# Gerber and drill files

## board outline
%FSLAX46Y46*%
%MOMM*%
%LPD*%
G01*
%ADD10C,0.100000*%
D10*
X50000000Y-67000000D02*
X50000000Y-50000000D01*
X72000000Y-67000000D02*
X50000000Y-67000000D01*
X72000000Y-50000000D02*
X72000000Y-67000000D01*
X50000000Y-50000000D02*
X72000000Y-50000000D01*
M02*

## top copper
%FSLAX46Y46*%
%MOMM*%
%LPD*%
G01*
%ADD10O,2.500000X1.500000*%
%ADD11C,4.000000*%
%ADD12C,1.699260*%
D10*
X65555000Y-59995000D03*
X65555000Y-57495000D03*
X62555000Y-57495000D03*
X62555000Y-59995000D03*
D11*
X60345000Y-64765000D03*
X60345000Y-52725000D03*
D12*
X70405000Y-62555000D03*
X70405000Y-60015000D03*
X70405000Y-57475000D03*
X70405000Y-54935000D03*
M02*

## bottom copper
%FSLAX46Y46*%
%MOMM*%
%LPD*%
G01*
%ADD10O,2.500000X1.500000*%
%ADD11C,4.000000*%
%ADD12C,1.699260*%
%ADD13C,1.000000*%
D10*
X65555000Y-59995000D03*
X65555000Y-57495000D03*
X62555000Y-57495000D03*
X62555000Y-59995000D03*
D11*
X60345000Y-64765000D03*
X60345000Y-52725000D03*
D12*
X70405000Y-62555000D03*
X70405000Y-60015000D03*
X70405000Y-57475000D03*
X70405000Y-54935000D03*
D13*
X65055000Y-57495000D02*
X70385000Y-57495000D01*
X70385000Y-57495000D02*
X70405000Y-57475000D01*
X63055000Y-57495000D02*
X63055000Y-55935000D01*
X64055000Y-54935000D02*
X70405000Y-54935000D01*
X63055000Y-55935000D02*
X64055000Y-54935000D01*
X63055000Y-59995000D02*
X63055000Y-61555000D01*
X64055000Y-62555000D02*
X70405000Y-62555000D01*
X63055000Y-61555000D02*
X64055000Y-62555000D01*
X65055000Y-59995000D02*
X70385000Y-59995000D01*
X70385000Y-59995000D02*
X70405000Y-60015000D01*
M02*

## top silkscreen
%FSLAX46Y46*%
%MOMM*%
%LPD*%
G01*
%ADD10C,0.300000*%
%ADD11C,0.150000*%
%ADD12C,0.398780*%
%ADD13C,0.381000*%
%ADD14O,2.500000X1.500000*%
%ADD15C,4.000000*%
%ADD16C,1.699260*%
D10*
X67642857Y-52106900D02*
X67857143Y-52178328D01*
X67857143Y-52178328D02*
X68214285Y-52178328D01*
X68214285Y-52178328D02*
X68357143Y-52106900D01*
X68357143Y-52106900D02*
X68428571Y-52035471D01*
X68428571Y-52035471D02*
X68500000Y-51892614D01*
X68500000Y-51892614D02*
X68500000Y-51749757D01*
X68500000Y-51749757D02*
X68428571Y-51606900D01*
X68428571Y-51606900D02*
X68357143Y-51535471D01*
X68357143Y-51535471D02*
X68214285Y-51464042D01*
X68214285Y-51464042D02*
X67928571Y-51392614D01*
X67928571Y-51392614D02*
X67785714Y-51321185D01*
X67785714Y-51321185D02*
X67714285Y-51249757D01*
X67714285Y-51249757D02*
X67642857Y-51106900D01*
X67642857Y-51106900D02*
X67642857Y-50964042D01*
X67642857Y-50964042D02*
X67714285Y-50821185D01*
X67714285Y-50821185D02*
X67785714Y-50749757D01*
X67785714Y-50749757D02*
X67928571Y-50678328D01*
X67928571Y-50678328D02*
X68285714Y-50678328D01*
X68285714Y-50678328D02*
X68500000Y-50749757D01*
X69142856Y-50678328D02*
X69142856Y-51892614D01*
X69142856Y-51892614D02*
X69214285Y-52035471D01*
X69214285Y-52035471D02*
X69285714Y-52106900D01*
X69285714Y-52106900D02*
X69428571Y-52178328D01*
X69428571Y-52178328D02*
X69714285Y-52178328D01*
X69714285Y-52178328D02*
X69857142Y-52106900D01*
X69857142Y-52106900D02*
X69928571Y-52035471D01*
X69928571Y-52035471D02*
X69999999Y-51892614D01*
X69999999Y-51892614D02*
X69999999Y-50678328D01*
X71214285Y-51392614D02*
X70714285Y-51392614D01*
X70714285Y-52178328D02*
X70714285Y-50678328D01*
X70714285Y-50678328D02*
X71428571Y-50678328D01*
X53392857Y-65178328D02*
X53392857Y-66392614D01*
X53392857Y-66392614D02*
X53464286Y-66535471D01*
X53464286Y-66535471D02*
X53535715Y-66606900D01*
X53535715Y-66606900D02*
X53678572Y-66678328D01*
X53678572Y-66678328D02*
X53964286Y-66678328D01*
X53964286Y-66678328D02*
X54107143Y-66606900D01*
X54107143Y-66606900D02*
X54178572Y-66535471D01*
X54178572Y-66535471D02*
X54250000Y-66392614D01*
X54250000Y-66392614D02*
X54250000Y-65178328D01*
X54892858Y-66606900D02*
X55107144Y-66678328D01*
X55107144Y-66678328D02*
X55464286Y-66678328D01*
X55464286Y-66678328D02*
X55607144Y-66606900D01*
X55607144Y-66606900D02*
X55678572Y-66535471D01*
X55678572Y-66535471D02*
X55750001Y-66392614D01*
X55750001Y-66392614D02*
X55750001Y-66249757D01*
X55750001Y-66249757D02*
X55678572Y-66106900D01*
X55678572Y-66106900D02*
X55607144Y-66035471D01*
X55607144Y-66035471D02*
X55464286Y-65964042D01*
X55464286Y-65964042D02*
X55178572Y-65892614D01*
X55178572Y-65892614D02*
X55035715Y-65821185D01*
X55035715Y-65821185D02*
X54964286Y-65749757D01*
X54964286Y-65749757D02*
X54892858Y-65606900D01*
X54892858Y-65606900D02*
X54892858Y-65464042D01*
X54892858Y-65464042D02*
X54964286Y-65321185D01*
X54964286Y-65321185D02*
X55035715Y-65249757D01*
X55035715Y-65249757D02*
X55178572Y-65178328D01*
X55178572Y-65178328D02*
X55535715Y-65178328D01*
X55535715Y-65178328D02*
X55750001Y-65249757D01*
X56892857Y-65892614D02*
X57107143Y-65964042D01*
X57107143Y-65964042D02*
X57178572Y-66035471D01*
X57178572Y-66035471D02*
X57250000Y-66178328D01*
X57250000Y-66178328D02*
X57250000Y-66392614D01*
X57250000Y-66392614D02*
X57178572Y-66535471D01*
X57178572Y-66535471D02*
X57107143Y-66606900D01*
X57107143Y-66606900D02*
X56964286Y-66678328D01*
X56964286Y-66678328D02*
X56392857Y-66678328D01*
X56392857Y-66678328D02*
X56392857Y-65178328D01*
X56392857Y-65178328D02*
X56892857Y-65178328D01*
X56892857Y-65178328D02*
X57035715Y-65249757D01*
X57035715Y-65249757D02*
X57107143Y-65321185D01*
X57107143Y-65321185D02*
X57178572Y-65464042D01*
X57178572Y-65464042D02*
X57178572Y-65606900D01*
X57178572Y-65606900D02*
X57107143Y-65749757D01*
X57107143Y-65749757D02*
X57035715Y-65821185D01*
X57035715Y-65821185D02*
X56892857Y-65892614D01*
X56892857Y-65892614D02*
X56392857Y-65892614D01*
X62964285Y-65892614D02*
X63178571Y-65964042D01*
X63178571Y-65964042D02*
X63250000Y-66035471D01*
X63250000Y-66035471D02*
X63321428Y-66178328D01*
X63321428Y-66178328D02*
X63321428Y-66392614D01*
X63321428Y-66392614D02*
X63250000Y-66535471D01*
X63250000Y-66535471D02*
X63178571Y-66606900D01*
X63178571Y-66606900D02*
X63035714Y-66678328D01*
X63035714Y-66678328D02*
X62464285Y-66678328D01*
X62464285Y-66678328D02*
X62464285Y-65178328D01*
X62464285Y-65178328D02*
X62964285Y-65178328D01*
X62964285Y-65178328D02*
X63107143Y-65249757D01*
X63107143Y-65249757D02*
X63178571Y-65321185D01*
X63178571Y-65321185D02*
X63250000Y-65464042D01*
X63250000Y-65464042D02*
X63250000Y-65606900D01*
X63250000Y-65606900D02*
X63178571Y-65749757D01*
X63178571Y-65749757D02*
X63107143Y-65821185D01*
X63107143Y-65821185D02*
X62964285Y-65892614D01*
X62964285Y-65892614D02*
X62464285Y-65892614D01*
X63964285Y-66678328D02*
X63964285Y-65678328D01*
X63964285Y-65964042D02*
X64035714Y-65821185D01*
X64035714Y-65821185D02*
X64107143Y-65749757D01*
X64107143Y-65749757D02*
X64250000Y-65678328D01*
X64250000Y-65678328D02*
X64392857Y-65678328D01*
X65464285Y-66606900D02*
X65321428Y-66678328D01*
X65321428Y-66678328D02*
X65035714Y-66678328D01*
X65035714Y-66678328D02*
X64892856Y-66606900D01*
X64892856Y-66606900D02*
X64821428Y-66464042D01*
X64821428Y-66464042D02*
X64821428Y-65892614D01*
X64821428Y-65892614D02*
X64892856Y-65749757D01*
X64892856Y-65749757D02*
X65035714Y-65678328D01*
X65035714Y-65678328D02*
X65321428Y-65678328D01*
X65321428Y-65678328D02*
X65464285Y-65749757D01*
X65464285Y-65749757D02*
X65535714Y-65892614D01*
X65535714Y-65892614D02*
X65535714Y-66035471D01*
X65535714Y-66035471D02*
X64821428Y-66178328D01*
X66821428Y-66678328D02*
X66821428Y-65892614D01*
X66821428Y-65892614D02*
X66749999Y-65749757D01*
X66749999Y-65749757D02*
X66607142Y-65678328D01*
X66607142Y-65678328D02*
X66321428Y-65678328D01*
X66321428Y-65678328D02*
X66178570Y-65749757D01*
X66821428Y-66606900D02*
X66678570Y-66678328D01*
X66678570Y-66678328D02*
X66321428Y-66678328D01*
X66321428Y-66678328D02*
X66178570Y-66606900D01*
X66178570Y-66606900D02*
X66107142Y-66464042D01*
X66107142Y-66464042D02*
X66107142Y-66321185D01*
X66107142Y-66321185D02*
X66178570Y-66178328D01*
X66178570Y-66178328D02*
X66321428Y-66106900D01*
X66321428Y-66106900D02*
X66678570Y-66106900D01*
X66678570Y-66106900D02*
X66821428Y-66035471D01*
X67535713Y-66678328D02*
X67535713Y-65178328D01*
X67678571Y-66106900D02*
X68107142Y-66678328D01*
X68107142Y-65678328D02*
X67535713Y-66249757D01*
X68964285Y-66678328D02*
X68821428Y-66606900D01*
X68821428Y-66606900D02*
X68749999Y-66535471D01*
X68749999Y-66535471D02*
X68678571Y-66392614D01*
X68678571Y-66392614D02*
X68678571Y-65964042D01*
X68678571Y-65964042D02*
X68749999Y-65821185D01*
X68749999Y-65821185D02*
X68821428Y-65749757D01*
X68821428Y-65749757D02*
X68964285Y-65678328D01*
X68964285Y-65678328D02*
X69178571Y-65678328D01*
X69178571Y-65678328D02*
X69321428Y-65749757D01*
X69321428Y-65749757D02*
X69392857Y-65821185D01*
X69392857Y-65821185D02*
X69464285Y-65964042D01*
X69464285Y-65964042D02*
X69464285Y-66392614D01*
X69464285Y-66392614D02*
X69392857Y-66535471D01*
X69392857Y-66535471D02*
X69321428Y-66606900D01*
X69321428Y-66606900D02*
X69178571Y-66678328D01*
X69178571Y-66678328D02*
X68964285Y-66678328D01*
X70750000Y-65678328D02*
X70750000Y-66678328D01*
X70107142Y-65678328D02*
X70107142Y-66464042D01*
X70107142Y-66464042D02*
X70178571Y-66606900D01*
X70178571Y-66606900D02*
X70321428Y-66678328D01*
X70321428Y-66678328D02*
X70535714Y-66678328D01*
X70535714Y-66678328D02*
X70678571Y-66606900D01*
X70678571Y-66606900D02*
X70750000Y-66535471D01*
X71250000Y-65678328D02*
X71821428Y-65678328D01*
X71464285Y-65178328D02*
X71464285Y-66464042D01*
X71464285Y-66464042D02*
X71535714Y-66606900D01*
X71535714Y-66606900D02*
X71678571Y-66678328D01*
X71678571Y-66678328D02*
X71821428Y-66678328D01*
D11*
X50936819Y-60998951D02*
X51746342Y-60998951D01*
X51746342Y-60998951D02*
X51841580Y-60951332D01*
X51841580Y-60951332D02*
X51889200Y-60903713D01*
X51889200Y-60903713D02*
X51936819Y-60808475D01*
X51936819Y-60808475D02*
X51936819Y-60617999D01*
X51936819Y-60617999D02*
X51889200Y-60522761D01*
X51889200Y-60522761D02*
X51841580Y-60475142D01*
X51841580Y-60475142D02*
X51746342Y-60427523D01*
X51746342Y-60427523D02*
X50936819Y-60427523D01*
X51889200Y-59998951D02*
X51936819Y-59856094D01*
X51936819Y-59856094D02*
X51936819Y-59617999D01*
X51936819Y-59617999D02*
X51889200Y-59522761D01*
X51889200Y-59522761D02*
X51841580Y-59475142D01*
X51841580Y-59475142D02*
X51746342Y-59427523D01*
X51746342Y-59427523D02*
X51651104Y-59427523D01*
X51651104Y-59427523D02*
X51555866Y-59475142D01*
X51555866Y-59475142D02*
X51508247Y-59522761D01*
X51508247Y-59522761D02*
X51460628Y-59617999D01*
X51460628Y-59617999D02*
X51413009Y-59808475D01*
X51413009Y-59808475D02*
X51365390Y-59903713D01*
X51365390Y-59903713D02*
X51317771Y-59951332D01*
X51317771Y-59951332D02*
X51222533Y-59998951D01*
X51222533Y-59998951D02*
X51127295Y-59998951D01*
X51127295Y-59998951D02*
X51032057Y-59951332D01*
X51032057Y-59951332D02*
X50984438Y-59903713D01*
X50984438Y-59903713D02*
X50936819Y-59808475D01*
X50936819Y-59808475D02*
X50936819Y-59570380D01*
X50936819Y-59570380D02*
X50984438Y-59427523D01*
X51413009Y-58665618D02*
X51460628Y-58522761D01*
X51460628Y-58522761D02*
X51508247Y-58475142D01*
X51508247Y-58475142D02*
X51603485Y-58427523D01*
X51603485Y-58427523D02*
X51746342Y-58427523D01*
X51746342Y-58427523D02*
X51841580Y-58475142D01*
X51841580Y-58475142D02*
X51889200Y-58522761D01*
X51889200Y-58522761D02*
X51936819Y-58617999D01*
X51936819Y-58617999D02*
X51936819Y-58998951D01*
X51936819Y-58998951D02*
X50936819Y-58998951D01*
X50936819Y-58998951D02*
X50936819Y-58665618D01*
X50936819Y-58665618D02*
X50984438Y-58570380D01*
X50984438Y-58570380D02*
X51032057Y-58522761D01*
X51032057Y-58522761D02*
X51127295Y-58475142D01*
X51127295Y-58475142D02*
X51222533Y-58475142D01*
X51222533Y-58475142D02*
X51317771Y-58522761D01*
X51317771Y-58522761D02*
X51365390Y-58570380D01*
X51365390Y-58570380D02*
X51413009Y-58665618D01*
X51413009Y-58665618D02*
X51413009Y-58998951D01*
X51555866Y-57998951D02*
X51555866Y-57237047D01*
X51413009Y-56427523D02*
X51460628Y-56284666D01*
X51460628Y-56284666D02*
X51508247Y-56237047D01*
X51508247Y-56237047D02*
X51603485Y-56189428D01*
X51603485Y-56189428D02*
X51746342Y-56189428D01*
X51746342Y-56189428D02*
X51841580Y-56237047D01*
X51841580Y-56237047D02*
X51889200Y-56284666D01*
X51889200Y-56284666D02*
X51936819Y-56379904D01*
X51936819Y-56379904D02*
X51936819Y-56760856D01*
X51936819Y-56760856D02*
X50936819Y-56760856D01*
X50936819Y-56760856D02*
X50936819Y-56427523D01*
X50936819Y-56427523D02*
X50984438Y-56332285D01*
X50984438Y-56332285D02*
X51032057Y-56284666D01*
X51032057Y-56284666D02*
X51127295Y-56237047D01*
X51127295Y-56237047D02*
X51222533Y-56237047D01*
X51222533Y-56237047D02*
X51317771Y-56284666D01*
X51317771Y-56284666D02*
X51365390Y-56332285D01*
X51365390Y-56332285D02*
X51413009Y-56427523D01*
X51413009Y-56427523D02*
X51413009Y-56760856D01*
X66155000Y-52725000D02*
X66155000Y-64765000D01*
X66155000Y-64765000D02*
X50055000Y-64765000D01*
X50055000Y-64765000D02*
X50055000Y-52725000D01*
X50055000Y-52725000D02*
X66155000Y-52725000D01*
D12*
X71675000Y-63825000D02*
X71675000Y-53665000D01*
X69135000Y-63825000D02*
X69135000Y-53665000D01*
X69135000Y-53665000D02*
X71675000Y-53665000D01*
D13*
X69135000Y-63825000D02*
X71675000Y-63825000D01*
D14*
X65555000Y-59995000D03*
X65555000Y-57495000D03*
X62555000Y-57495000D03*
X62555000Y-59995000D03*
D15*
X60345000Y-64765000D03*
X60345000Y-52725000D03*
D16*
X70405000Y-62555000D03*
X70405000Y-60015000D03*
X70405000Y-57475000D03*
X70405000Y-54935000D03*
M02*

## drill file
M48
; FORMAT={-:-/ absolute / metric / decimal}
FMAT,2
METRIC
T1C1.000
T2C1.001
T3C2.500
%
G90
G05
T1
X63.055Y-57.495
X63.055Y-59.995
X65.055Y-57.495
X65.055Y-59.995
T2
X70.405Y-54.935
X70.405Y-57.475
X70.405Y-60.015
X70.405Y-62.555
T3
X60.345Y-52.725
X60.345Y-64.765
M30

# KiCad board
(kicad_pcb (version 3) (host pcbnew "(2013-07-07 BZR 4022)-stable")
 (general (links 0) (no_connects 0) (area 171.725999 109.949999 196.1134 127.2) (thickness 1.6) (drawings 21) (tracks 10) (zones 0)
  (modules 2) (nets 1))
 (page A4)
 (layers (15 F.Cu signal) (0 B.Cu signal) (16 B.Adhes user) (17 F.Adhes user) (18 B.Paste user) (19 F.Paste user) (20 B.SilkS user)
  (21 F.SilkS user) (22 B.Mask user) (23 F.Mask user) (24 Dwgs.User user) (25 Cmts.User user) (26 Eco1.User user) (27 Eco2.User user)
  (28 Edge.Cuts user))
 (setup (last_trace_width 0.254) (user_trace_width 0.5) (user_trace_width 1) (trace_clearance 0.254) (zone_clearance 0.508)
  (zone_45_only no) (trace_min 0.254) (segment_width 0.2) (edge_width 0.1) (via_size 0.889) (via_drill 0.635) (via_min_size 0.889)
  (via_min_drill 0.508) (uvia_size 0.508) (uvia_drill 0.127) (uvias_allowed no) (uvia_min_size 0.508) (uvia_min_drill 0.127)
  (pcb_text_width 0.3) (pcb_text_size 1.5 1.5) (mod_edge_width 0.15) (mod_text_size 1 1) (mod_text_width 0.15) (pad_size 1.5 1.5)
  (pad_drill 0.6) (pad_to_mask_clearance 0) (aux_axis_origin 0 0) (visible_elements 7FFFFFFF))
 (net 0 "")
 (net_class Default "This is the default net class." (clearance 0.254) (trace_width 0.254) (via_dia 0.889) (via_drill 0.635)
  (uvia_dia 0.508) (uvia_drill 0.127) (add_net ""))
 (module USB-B (layer F.Cu) (at 64.055 58.745 270)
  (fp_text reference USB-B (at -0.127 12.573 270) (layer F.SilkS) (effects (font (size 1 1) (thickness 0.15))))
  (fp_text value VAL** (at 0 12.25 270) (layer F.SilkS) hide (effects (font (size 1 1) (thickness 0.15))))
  (fp_line (start -6.02 -2.1) (end 6.02 -2.1) (layer F.SilkS) (width 0.15))
  (fp_line (start 6.02 -2.1) (end 6.02 14) (layer F.SilkS) (width 0.15))
  (fp_line (start 6.02 14) (end -6.02 14) (layer F.SilkS) (width 0.15))
  (fp_line (start -6.02 14) (end -6.02 -2.1) (layer F.SilkS) (width 0.15))
  (pad 1 thru_hole oval (at 1.25 -1 270) (size 1.5 2.5) (drill 1 (offset 0 -0.5)) (layers *.Cu *.Mask F.SilkS))
  (pad 2 thru_hole oval (at -1.25 -1 270) (size 1.5 2.5) (drill 1 (offset 0 -0.5)) (layers *.Cu *.Mask F.SilkS))
  (pad 3 thru_hole oval (at -1.25 1 270) (size 1.5 2.5) (drill 1 (offset 0 0.5)) (layers *.Cu *.Mask F.SilkS))
  (pad 4 thru_hole oval (at 1.25 1 270) (size 1.5 2.5) (drill 1 (offset 0 0.5)) (layers *.Cu *.Mask F.SilkS))
  (pad "" thru_hole circle (at 6.02 3.71 270) (size 4 4) (drill 2.5) (layers *.Cu *.Mask F.SilkS))
  (pad "" thru_hole circle (at -6.02 3.71 270) (size 4 4) (drill 2.5) (layers *.Cu *.Mask F.SilkS)))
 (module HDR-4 (layer F.Cu) (at 70.405 58.745 90)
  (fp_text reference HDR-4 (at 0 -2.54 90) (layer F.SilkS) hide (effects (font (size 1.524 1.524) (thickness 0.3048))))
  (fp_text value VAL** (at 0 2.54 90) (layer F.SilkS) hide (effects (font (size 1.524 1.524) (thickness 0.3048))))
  (fp_line (start -5.08 1.27) (end 5.08 1.27) (layer F.SilkS) (width 0.39878))
  (fp_line (start -5.08 -1.27) (end 5.08 -1.27) (layer F.SilkS) (width 0.39878))
  (fp_line (start 5.08 -1.27) (end 5.08 1.27) (layer F.SilkS) (width 0.39878))
  (fp_line (start -5.08 -1.27) (end -5.08 1.27) (layer F.SilkS) (width 0.381))
  (pad 1 thru_hole circle (at -3.81 0 90) (size 1.69926 1.69926) (drill 1.00076) (layers *.Cu *.Mask F.SilkS))
  (pad 2 thru_hole circle (at -1.27 0 90) (size 1.69926 1.69926) (drill 1.00076) (layers *.Cu *.Mask F.SilkS))
  (pad 3 thru_hole circle (at 1.27 0 90) (size 1.69926 1.69926) (drill 1.00076) (layers *.Cu *.Mask F.SilkS))
  (pad 4 thru_hole circle (at 3.81 0 90) (size 1.69926 1.69926) (drill 1.00076) (layers *.Cu *.Mask F.SilkS)))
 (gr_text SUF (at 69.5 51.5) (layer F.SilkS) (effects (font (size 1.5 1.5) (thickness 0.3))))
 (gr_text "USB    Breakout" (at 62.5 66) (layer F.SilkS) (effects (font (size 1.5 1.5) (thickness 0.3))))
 (gr_line (start 50 67) (end 50 50) (angle 90) (layer Edge.Cuts) (width 0.1))
 (gr_line (start 72 67) (end 50 67) (angle 90) (layer Edge.Cuts) (width 0.1))
 (gr_line (start 72 50) (end 72 67) (angle 90) (layer Edge.Cuts) (width 0.1))
 (gr_line (start 50 50) (end 72 50) (angle 90) (layer Edge.Cuts) (width 0.1))
 (segment (start 65.055 57.495) (end 70.385 57.495) (width 1) (layer B.Cu) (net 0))
 (segment (start 70.385 57.495) (end 70.405 57.475) (width 1) (layer B.Cu) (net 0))
 (segment (start 63.055 57.495) (end 63.055 55.935) (width 1) (layer B.Cu) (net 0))
 (segment (start 64.055 54.935) (end 70.405 54.935) (width 1) (layer B.Cu) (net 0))
 (segment (start 63.055 55.935) (end 64.055 54.935) (width 1) (layer B.Cu) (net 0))
 (segment (start 63.055 59.995) (end 63.055 61.555) (width 1) (layer B.Cu) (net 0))
 (segment (start 64.055 62.555) (end 70.405 62.555) (width 1) (layer B.Cu) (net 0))
 (segment (start 63.055 61.555) (end 64.055 62.555) (width 1) (layer B.Cu) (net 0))
 (segment (start 65.055 59.995) (end 70.385 59.995) (width 1) (layer B.Cu) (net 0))
 (segment (start 70.385 59.995) (end 70.405 60.015) (width 1) (layer B.Cu) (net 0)))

